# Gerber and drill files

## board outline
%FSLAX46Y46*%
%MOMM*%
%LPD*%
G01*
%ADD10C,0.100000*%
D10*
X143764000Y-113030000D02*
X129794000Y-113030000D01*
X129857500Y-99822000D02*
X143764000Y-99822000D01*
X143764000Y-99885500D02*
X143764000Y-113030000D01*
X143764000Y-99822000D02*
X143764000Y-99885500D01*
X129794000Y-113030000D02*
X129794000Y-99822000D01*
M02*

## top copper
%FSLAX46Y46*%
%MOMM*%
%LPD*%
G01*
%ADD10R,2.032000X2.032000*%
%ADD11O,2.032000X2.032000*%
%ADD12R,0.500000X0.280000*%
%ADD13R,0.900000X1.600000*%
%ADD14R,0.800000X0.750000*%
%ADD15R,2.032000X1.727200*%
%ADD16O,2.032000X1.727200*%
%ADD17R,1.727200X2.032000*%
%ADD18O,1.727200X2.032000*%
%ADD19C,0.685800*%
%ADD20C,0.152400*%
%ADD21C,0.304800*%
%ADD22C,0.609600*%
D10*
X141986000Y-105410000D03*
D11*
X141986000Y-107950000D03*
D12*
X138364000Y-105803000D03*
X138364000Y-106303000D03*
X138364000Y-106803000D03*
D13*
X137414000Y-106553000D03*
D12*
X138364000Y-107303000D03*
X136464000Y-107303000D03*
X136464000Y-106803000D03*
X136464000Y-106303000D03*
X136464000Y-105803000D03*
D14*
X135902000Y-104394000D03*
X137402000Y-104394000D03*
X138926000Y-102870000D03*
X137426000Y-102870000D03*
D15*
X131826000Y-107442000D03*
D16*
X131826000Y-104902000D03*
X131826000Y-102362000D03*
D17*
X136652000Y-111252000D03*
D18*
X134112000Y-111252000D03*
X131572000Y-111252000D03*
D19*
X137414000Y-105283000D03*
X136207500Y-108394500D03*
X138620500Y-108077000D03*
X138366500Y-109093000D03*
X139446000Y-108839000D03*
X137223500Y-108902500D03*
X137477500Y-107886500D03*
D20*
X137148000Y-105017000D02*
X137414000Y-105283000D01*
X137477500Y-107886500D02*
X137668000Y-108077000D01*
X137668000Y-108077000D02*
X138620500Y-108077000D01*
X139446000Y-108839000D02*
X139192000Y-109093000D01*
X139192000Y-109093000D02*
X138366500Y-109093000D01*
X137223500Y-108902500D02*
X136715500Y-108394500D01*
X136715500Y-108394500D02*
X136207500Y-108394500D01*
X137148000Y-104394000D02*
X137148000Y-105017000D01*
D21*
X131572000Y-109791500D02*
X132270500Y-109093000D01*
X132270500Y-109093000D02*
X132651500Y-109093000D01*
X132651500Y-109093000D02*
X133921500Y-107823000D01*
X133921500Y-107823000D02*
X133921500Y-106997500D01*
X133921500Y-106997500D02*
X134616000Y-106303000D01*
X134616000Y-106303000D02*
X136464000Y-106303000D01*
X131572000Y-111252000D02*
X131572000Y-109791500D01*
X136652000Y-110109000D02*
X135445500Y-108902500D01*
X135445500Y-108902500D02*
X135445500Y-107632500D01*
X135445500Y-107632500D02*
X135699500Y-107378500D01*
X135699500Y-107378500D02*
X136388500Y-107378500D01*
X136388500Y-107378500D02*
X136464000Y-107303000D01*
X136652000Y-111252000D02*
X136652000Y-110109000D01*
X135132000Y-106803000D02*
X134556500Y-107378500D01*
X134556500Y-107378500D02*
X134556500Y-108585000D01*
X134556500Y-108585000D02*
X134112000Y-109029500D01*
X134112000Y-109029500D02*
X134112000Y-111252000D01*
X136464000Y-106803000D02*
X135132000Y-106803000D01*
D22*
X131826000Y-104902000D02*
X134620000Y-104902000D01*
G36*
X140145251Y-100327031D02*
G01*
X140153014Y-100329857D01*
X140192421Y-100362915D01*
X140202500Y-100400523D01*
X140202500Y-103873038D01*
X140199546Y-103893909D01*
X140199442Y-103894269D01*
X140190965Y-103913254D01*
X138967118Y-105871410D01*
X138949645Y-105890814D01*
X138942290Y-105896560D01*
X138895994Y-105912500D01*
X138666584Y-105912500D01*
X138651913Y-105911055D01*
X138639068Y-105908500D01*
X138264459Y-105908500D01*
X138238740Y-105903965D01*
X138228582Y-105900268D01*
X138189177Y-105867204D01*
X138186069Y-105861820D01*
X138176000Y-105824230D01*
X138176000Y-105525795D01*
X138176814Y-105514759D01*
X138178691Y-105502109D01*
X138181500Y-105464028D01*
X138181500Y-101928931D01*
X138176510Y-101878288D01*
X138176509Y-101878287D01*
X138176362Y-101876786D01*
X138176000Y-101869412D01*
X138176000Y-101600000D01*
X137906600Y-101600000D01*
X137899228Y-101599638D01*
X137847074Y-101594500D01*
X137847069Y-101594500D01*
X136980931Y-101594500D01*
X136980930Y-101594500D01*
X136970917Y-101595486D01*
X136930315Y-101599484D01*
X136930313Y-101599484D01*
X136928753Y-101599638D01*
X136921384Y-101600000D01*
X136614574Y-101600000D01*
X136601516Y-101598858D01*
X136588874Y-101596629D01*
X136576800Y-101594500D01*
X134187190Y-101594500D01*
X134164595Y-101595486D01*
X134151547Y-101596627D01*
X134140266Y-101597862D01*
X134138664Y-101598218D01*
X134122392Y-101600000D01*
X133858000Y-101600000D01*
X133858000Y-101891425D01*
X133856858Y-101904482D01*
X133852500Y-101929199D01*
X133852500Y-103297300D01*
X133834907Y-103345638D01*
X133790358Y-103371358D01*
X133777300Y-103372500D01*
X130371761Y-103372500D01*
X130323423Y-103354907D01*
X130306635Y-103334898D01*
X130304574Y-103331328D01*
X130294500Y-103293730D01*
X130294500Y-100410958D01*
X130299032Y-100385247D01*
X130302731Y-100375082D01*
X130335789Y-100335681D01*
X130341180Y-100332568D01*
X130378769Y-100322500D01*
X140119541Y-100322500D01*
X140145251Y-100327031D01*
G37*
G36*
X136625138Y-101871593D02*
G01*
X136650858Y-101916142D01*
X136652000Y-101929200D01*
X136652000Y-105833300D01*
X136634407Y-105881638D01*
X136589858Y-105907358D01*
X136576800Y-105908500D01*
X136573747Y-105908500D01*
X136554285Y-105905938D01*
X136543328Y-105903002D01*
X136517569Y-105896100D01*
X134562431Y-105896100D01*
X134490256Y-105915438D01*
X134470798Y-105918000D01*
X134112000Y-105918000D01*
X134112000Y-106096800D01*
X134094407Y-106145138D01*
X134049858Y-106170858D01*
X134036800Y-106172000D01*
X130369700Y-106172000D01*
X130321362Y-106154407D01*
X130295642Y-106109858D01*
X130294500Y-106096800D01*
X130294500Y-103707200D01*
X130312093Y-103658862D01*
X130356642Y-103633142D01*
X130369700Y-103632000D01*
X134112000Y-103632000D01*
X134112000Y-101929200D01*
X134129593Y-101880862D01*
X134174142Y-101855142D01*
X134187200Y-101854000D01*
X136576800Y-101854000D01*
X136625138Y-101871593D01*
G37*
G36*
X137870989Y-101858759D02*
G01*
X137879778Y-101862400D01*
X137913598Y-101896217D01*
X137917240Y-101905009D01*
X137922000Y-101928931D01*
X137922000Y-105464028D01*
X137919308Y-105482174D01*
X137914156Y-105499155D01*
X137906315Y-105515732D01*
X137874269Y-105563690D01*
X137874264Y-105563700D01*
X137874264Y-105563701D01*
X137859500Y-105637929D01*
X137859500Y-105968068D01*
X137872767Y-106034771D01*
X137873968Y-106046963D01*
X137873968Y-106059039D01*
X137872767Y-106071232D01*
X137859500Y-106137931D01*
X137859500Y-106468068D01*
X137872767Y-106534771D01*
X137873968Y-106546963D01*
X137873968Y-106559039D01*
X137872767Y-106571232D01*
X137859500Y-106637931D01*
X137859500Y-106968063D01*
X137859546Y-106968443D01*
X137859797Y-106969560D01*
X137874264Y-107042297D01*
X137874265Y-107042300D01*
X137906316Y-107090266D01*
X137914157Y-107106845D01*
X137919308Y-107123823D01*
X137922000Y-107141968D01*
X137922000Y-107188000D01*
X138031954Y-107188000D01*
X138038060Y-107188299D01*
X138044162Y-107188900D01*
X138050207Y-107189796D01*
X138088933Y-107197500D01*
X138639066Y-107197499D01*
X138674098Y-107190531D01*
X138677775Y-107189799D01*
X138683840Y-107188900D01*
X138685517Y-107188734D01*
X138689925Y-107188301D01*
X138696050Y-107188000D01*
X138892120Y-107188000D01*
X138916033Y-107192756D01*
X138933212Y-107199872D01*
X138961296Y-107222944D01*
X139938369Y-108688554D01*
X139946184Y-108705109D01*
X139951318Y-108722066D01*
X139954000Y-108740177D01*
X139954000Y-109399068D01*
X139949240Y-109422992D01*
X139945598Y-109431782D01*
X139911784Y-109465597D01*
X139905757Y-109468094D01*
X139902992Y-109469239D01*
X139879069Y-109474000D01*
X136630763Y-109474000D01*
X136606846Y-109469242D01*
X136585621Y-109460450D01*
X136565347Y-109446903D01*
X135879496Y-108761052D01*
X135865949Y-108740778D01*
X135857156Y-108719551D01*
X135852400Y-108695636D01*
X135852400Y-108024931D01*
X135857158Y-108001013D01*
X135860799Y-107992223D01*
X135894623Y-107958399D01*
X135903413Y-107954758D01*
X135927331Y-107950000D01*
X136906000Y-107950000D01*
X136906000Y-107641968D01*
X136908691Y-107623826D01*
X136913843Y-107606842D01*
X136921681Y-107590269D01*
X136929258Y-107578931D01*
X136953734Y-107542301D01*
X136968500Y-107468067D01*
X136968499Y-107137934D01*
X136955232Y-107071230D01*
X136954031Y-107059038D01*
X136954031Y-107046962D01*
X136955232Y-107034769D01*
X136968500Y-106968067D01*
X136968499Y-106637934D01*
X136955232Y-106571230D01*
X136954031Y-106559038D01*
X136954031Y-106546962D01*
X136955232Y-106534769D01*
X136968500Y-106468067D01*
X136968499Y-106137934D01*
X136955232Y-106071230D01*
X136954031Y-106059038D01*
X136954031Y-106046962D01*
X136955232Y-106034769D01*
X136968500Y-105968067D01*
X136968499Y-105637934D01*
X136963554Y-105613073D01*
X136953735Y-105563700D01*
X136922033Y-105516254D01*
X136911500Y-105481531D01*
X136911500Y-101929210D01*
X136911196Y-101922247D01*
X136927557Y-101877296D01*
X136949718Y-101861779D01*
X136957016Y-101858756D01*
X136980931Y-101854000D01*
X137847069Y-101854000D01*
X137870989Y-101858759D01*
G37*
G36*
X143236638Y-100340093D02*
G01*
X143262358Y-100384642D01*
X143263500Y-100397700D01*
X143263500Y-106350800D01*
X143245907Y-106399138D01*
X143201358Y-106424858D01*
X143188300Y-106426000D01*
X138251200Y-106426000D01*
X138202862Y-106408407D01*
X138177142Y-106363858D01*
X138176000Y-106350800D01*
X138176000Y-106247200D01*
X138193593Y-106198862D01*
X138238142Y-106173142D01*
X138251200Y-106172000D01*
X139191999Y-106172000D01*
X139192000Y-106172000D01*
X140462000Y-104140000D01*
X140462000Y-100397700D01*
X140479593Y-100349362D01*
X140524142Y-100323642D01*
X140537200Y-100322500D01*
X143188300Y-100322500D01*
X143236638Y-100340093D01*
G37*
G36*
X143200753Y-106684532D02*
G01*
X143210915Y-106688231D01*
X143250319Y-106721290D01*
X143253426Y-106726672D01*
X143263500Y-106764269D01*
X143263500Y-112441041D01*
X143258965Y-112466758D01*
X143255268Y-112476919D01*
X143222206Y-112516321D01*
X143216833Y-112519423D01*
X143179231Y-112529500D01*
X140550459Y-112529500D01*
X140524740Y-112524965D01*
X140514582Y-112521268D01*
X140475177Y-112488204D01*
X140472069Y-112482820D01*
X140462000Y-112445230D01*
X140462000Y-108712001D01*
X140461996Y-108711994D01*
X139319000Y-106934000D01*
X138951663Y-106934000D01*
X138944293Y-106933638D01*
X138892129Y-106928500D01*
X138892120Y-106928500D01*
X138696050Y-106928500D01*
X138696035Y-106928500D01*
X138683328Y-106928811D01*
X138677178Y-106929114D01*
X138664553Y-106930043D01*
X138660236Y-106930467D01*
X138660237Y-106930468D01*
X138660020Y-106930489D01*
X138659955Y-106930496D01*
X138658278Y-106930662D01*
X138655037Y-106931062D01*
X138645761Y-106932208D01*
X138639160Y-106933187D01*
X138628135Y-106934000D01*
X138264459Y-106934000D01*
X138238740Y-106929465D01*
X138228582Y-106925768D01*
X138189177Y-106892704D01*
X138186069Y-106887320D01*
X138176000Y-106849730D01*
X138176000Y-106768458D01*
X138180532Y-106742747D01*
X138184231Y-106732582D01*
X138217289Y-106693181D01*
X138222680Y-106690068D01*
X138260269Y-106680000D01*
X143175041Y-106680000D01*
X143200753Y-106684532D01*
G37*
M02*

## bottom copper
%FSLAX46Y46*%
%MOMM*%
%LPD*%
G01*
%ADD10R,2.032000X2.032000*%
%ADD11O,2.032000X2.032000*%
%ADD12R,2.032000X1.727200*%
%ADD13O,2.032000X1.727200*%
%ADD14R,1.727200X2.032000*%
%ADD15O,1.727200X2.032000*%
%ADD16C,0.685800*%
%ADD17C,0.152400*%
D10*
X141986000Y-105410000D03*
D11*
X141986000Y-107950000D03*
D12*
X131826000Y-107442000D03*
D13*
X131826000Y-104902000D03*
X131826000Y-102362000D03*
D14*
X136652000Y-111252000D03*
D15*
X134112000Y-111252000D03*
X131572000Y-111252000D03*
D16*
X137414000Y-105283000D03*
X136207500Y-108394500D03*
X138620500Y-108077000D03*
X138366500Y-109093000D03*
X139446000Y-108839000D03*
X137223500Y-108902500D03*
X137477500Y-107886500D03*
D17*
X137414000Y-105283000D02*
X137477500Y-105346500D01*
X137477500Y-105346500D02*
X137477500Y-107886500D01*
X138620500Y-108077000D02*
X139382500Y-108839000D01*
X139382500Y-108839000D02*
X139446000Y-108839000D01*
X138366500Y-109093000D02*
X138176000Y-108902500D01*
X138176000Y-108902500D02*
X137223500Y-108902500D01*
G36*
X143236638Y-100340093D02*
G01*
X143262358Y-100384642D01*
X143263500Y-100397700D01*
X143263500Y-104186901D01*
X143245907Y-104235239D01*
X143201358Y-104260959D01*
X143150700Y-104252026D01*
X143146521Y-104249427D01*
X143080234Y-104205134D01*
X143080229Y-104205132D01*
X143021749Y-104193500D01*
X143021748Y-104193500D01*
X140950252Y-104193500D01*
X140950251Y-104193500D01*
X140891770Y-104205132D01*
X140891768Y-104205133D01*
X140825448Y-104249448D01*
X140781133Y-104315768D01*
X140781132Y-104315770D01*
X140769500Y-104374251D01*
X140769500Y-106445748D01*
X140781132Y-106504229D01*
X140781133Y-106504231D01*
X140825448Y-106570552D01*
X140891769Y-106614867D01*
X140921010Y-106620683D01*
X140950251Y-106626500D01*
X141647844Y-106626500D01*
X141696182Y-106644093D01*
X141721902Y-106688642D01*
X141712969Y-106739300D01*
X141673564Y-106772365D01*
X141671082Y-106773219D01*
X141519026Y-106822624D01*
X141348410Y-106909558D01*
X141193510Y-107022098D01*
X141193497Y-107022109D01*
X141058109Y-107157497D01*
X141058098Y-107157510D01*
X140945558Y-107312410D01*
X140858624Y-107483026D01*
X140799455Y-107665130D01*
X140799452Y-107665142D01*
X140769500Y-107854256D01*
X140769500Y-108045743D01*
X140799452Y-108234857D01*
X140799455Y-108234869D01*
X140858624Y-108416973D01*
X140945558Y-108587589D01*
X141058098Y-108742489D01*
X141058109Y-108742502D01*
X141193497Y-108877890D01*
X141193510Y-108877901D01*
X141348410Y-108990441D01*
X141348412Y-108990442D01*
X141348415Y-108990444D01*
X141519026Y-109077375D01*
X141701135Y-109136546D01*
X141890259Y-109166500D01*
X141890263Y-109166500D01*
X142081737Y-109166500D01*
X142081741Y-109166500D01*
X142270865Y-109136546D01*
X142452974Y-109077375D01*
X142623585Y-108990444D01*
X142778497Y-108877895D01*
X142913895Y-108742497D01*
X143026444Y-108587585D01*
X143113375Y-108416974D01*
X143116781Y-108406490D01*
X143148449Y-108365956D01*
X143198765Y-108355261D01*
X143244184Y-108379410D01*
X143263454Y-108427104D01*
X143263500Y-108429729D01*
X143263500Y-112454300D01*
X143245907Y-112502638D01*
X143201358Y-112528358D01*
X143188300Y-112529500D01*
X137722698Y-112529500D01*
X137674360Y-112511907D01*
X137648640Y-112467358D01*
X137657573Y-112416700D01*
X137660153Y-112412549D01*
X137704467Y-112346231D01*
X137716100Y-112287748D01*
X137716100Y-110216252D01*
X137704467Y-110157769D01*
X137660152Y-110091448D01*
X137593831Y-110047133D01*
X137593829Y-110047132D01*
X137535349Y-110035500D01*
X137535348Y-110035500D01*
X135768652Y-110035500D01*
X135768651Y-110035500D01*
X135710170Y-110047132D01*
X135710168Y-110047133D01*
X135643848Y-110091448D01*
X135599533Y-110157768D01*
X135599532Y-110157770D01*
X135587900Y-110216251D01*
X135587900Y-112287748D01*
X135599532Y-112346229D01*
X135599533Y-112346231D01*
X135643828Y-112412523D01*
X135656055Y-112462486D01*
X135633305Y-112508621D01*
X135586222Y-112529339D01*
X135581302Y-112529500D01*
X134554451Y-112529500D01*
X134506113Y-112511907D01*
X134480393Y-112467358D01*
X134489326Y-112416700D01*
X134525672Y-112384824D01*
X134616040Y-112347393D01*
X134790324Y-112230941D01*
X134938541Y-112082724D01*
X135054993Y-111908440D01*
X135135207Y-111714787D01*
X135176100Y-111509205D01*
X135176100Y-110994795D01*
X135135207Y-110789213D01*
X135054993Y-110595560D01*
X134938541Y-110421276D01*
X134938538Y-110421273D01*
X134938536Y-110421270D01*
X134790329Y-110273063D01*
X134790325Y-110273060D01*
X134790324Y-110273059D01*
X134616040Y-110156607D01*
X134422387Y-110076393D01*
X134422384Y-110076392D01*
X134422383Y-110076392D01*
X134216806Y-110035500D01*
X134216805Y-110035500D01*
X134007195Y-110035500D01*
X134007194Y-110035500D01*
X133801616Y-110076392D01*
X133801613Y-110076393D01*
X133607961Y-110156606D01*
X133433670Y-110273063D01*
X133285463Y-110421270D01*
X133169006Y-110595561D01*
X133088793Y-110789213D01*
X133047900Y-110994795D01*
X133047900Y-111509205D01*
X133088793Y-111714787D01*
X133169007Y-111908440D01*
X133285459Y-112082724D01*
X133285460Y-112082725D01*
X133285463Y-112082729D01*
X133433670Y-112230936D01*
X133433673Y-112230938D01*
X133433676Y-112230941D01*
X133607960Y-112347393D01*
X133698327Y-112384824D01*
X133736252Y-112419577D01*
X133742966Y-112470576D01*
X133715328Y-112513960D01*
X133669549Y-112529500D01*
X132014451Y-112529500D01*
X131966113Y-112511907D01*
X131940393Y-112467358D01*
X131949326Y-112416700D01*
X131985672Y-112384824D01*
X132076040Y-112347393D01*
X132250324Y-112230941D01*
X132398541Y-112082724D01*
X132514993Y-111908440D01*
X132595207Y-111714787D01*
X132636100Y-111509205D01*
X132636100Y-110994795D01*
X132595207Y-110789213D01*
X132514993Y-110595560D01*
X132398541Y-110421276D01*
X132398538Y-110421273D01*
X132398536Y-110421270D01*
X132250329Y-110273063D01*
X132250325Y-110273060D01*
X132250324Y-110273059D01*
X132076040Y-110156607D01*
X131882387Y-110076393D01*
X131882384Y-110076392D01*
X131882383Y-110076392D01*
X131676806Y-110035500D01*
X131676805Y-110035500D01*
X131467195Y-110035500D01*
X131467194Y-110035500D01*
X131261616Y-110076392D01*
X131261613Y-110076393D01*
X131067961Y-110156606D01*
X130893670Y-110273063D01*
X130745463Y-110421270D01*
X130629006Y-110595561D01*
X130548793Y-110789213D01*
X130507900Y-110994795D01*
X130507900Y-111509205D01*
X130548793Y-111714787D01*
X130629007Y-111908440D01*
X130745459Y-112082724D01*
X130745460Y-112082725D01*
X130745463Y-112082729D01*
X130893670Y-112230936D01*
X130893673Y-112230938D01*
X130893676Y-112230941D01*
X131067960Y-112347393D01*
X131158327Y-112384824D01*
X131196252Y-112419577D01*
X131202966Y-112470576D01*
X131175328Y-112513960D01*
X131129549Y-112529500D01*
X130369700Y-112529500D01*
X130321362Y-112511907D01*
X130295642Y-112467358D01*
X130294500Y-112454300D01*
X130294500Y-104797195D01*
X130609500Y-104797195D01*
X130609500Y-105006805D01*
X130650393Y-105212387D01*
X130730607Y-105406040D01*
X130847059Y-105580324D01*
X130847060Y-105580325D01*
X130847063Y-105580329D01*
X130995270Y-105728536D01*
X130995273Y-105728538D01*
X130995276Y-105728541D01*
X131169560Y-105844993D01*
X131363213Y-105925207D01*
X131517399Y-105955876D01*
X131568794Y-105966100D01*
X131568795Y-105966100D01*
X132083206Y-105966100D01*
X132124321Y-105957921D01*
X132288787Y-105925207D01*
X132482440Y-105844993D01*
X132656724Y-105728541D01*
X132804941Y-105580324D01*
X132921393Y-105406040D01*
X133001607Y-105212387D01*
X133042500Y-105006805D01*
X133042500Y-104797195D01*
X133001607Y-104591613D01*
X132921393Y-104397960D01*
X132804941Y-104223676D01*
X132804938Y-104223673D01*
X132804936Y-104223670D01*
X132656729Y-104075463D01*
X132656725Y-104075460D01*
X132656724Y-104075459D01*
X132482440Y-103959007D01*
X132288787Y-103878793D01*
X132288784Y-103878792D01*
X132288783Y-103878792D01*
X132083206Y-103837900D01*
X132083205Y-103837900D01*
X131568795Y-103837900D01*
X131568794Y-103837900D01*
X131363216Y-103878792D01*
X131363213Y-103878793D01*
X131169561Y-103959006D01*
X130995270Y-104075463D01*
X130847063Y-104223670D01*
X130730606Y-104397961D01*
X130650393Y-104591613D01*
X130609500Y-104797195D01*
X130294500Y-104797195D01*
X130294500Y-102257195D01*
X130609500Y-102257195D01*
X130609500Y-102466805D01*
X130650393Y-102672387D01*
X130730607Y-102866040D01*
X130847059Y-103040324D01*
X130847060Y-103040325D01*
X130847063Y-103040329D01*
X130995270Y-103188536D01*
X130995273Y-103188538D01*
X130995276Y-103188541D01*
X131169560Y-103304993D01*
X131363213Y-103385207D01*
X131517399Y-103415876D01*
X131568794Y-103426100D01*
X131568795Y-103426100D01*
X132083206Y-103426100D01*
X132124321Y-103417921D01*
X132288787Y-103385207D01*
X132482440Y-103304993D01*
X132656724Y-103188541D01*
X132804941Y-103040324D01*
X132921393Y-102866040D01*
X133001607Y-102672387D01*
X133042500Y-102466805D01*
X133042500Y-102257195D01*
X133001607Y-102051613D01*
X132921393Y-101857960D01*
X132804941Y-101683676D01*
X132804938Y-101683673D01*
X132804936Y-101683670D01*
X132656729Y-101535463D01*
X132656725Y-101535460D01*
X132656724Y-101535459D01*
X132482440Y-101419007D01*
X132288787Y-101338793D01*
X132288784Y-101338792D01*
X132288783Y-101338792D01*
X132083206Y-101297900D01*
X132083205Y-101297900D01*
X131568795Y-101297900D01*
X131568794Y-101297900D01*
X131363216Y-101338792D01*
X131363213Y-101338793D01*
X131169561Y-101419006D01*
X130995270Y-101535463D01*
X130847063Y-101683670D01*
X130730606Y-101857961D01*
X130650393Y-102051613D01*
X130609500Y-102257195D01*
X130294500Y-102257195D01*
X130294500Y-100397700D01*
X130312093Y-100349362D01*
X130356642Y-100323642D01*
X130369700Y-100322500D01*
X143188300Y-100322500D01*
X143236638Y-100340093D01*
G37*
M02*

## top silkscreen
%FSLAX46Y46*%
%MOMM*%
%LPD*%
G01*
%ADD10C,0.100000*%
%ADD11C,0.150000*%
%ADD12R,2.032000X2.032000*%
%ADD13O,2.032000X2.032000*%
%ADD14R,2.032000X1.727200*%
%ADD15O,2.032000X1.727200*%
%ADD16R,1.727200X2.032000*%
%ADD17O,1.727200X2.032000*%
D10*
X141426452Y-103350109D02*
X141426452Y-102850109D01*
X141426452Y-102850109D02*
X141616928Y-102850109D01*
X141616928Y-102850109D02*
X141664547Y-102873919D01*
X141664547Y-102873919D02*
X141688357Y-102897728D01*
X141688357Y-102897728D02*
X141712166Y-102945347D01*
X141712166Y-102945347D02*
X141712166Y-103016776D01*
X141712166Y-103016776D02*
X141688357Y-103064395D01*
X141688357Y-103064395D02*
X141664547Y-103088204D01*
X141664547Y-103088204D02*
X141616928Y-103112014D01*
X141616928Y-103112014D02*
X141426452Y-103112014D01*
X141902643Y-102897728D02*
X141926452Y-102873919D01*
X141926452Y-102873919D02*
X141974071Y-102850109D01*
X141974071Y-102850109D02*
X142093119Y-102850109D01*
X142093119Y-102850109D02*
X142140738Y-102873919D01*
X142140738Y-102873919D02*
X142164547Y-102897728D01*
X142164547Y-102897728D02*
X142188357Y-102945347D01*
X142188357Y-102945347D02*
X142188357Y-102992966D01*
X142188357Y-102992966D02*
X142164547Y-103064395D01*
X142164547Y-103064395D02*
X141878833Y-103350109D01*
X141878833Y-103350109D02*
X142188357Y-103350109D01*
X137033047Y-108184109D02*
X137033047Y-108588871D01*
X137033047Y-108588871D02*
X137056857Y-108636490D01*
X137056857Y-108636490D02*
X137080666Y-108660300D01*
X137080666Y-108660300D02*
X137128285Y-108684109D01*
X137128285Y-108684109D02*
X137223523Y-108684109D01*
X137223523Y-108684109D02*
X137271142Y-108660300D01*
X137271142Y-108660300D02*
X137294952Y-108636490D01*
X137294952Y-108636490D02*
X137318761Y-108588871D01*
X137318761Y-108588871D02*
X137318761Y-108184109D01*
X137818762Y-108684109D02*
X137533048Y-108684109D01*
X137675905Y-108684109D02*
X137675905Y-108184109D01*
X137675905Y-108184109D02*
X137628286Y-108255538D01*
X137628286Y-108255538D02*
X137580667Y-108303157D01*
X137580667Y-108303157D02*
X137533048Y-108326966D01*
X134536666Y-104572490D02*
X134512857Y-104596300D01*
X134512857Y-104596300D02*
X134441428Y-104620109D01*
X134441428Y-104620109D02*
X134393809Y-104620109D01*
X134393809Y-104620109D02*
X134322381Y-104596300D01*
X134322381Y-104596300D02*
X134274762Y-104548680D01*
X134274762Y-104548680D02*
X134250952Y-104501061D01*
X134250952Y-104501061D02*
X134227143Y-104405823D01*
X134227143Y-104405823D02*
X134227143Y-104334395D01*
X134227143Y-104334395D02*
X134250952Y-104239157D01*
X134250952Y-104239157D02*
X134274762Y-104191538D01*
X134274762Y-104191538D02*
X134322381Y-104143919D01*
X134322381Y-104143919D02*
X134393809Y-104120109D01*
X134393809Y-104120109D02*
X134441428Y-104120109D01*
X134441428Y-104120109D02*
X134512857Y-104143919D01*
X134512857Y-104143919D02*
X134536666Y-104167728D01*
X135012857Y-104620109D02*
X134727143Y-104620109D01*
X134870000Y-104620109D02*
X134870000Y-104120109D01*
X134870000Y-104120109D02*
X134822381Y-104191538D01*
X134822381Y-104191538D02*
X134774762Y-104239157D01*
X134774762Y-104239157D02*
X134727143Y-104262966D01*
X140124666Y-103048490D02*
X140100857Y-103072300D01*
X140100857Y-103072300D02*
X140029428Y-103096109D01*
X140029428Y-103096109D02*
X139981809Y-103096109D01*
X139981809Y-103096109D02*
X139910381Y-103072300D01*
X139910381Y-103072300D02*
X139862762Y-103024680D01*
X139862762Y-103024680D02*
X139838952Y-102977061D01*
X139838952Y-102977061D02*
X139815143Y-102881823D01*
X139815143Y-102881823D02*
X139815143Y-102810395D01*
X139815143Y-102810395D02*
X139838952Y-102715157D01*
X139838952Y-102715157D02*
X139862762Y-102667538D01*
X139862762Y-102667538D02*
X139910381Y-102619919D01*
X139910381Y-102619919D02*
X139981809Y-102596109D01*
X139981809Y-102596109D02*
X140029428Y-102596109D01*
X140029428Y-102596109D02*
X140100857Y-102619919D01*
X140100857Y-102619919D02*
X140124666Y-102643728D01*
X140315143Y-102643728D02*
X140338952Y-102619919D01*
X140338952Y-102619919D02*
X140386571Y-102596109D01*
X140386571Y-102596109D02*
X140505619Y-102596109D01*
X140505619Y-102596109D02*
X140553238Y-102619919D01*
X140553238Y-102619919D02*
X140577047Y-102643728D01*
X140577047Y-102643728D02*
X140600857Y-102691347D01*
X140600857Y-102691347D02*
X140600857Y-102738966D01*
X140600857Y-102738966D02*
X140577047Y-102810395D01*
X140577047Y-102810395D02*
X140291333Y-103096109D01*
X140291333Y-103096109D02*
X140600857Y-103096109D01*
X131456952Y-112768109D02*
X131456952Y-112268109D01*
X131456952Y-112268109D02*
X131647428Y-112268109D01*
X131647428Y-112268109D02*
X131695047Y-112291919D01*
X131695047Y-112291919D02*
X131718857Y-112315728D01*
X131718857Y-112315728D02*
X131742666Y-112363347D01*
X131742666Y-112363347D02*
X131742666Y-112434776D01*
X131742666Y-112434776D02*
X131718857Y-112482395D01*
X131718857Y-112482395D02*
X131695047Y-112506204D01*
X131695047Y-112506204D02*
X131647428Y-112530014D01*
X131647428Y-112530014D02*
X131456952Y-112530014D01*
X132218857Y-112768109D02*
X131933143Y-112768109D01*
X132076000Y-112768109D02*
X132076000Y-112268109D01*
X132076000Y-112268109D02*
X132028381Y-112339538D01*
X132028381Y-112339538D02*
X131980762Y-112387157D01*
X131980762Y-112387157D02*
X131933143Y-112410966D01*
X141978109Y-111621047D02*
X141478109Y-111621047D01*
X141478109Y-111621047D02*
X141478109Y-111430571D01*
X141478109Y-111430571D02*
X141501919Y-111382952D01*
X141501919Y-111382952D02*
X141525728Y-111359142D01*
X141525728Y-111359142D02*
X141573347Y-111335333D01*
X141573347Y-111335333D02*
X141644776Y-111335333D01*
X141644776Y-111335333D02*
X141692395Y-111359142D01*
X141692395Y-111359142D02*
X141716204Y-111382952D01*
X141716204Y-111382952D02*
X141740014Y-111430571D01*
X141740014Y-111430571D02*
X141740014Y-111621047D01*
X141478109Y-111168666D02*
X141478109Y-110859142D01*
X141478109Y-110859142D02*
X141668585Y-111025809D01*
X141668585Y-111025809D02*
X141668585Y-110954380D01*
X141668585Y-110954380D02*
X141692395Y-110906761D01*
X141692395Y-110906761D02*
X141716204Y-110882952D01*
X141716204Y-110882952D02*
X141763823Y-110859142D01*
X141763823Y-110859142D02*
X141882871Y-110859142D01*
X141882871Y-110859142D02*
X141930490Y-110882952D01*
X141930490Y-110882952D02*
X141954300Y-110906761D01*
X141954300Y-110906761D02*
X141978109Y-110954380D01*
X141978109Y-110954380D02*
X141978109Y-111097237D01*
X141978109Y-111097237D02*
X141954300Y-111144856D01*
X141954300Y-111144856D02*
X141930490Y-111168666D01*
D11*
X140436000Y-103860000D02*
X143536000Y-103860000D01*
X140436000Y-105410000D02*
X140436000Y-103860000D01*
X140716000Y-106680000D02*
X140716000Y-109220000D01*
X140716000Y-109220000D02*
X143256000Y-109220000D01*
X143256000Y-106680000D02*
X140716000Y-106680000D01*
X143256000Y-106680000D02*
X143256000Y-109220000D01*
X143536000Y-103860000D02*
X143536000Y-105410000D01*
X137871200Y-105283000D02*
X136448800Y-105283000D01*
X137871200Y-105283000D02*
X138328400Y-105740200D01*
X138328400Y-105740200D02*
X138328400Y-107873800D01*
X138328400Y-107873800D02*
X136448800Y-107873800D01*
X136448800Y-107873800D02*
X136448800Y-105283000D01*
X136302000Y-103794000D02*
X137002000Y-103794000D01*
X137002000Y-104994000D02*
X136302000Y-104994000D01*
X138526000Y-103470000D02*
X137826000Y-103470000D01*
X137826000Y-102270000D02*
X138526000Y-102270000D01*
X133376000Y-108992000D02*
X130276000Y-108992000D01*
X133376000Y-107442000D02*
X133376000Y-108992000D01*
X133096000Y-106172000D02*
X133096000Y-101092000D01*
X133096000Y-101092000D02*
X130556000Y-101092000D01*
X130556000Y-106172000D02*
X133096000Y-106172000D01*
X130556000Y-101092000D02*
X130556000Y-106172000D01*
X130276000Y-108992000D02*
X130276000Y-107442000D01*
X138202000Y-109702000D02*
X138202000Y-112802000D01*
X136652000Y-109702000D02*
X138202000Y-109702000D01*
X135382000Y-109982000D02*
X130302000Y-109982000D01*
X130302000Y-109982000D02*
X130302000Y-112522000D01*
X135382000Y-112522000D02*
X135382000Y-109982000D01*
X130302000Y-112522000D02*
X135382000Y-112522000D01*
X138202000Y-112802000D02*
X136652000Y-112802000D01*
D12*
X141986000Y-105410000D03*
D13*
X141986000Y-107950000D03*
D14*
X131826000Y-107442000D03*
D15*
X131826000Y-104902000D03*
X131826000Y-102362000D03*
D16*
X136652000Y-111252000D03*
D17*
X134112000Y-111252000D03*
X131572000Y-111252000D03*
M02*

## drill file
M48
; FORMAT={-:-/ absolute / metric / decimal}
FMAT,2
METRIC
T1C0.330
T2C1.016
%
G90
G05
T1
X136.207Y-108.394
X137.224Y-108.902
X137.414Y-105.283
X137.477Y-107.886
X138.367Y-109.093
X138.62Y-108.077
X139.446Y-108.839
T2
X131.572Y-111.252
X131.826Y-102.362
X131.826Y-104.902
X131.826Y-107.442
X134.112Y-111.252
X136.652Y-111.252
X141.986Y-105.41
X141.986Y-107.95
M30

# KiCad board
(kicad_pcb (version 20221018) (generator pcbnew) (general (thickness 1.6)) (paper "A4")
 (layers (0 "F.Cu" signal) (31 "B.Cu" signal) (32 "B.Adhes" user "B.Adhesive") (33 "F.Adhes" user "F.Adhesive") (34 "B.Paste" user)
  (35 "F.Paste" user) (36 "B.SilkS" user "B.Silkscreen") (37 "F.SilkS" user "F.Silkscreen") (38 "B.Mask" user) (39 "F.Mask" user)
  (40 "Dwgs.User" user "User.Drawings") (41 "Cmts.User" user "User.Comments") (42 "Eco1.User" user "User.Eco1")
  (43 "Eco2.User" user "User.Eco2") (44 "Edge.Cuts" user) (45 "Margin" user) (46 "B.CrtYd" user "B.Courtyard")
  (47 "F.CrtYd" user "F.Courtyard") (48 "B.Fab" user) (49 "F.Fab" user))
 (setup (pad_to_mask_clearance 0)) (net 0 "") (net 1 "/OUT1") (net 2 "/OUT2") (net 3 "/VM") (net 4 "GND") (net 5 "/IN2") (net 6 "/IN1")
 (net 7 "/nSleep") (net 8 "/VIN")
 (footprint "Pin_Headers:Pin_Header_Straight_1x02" (layer "F.Cu") (at 141.986 105.41)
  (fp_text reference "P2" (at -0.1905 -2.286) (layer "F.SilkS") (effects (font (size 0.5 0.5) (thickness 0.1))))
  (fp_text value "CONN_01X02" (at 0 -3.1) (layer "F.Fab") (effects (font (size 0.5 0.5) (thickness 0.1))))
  (fp_line (start -1.55 -1.55) (end 1.55 -1.55) (stroke (width 0.15) (type solid)) (layer "F.SilkS"))
  (fp_line (start -1.55 0) (end -1.55 -1.55) (stroke (width 0.15) (type solid)) (layer "F.SilkS"))
  (fp_line (start -1.27 1.27) (end -1.27 3.81) (stroke (width 0.15) (type solid)) (layer "F.SilkS"))
  (fp_line (start -1.27 3.81) (end 1.27 3.81) (stroke (width 0.15) (type solid)) (layer "F.SilkS"))
  (fp_line (start 1.27 1.27) (end -1.27 1.27) (stroke (width 0.15) (type solid)) (layer "F.SilkS"))
  (fp_line (start 1.27 1.27) (end 1.27 3.81) (stroke (width 0.15) (type solid)) (layer "F.SilkS"))
  (fp_line (start 1.55 -1.55) (end 1.55 0) (stroke (width 0.15) (type solid)) (layer "F.SilkS"))
  (pad "1" thru_hole rect (at 0 0) (size 2.032 2.032) (drill 1.016) (layers "*.Cu" "*.Mask" "F.SilkS") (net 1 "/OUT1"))
  (pad "2" thru_hole oval (at 0 2.54) (size 2.032 2.032) (drill 1.016) (layers "*.Cu" "*.Mask" "F.SilkS") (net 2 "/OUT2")))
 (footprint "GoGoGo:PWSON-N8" (layer "F.Cu") (at 137.414 106.553 -90)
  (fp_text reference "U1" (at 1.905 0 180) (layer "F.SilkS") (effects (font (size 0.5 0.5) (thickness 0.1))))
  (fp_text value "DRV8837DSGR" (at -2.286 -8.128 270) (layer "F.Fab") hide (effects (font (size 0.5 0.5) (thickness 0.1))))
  (fp_line (start -1.27 -0.4572) (end -1.27 0.9652) (stroke (width 0.15) (type solid)) (layer "F.SilkS"))
  (fp_line (start -1.27 -0.4572) (end -0.8128 -0.9144) (stroke (width 0.15) (type solid)) (layer "F.SilkS"))
  (fp_line (start -0.8128 -0.9144) (end 1.3208 -0.9144) (stroke (width 0.15) (type solid)) (layer "F.SilkS"))
  (fp_line (start 1.3208 -0.9144) (end 1.3208 0.9652) (stroke (width 0.15) (type solid)) (layer "F.SilkS"))
  (fp_line (start 1.3208 0.9652) (end -1.27 0.9652) (stroke (width 0.15) (type solid)) (layer "F.SilkS"))
  (pad "1" smd rect (at -0.75 -0.95 270) (size 0.28 0.5) (layers "F.Cu" "F.Paste" "F.Mask") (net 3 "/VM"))
  (pad "2" smd rect (at -0.25 -0.95 270) (size 0.28 0.5) (layers "F.Cu" "F.Paste" "F.Mask") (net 1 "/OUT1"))
  (pad "3" smd rect (at 0.25 -0.95 270) (size 0.28 0.5) (layers "F.Cu" "F.Paste" "F.Mask") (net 2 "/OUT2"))
  (pad "4" smd rect (at 0 0 270) (size 1.6 0.9) (layers "F.Cu" "F.Paste" "F.Mask") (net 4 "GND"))
  (pad "4" smd rect (at 0.75 -0.95 270) (size 0.28 0.5) (layers "F.Cu" "F.Paste" "F.Mask") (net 4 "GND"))
  (pad "5" smd rect (at 0.75 0.95 270) (size 0.28 0.5) (layers "F.Cu" "F.Paste" "F.Mask") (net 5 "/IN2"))
  (pad "6" smd rect (at 0.25 0.95 270) (size 0.28 0.5) (layers "F.Cu" "F.Paste" "F.Mask") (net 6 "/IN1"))
  (pad "7" smd rect (at -0.25 0.95 270) (size 0.28 0.5) (layers "F.Cu" "F.Paste" "F.Mask") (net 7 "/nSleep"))
  (pad "8" smd rect (at -0.75 0.95 270) (size 0.28 0.5) (layers "F.Cu" "F.Paste" "F.Mask") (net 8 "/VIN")))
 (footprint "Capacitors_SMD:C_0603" (layer "F.Cu") (at 136.652 104.394)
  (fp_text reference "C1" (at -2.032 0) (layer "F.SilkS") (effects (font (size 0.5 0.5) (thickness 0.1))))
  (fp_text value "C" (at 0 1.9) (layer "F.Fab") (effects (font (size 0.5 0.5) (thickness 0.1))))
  (fp_line (start -0.35 -0.6) (end 0.35 -0.6) (stroke (width 0.15) (type solid)) (layer "F.SilkS"))
  (fp_line (start 0.35 0.6) (end -0.35 0.6) (stroke (width 0.15) (type solid)) (layer "F.SilkS"))
  (pad "1" smd rect (at -0.75 0) (size 0.8 0.75) (layers "F.Cu" "F.Paste" "F.Mask") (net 8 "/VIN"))
  (pad "2" smd rect (at 0.75 0) (size 0.8 0.75) (layers "F.Cu" "F.Paste" "F.Mask") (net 4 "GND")))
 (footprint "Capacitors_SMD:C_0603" (layer "F.Cu") (at 138.176 102.87 180)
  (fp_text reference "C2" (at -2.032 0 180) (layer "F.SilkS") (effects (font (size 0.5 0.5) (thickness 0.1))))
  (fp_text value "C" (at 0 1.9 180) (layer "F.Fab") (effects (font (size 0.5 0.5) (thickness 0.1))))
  (fp_line (start -0.35 -0.6) (end 0.35 -0.6) (stroke (width 0.15) (type solid)) (layer "F.SilkS"))
  (fp_line (start 0.35 0.6) (end -0.35 0.6) (stroke (width 0.15) (type solid)) (layer "F.SilkS"))
  (pad "1" smd rect (at -0.75 0 180) (size 0.8 0.75) (layers "F.Cu" "F.Paste" "F.Mask") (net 3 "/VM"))
  (pad "2" smd rect (at 0.75 0 180) (size 0.8 0.75) (layers "F.Cu" "F.Paste" "F.Mask") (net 4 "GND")))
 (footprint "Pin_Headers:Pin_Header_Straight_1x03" (layer "F.Cu") (at 131.826 107.442 180)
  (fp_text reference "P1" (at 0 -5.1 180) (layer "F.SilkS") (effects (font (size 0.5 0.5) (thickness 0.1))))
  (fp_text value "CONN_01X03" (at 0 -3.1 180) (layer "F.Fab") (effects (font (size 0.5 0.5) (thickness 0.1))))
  (fp_line (start -1.55 -1.55) (end 1.55 -1.55) (stroke (width 0.15) (type solid)) (layer "F.SilkS"))
  (fp_line (start -1.55 0) (end -1.55 -1.55) (stroke (width 0.15) (type solid)) (layer "F.SilkS"))
  (fp_line (start -1.27 1.27) (end -1.27 6.35) (stroke (width 0.15) (type solid)) (layer "F.SilkS"))
  (fp_line (start -1.27 6.35) (end 1.27 6.35) (stroke (width 0.15) (type solid)) (layer "F.SilkS"))
  (fp_line (start 1.27 1.27) (end -1.27 1.27) (stroke (width 0.15) (type solid)) (layer "F.SilkS"))
  (fp_line (start 1.27 6.35) (end 1.27 1.27) (stroke (width 0.15) (type solid)) (layer "F.SilkS"))
  (fp_line (start 1.55 -1.55) (end 1.55 0) (stroke (width 0.15) (type solid)) (layer "F.SilkS"))
  (pad "1" thru_hole rect (at 0 0 180) (size 2.032 1.7272) (drill 1.016) (layers "*.Cu" "*.Mask" "F.SilkS") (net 4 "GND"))
  (pad "2" thru_hole oval (at 0 2.54 180) (size 2.032 1.7272) (drill 1.016) (layers "*.Cu" "*.Mask" "F.SilkS") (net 8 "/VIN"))
  (pad "3" thru_hole oval (at 0 5.08 180) (size 2.032 1.7272) (drill 1.016) (layers "*.Cu" "*.Mask" "F.SilkS") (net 3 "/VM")))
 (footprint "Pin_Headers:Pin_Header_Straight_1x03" (layer "F.Cu") (at 136.652 111.252 -90)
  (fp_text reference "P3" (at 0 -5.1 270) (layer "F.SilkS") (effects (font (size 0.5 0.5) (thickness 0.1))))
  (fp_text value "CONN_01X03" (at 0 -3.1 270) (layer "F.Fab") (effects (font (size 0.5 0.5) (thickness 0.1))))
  (fp_line (start -1.55 -1.55) (end 1.55 -1.55) (stroke (width 0.15) (type solid)) (layer "F.SilkS"))
  (fp_line (start -1.55 0) (end -1.55 -1.55) (stroke (width 0.15) (type solid)) (layer "F.SilkS"))
  (fp_line (start -1.27 1.27) (end -1.27 6.35) (stroke (width 0.15) (type solid)) (layer "F.SilkS"))
  (fp_line (start -1.27 6.35) (end 1.27 6.35) (stroke (width 0.15) (type solid)) (layer "F.SilkS"))
  (fp_line (start 1.27 1.27) (end -1.27 1.27) (stroke (width 0.15) (type solid)) (layer "F.SilkS"))
  (fp_line (start 1.27 6.35) (end 1.27 1.27) (stroke (width 0.15) (type solid)) (layer "F.SilkS"))
  (fp_line (start 1.55 -1.55) (end 1.55 0) (stroke (width 0.15) (type solid)) (layer "F.SilkS"))
  (pad "1" thru_hole rect (at 0 0 270) (size 2.032 1.7272) (drill 1.016) (layers "*.Cu" "*.Mask" "F.SilkS") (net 5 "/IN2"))
  (pad "2" thru_hole oval (at 0 2.54 270) (size 2.032 1.7272) (drill 1.016) (layers "*.Cu" "*.Mask" "F.SilkS") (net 6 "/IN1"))
  (pad "3" thru_hole oval (at 0 5.08 270) (size 2.032 1.7272) (drill 1.016) (layers "*.Cu" "*.Mask" "F.SilkS") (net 7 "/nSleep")))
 (gr_line (start 143.764 113.03) (end 129.794 113.03) (stroke (width 0.1) (type solid)) (layer "Edge.Cuts"))
 (gr_line (start 129.8575 99.822) (end 143.764 99.822) (stroke (width 0.1) (type solid)) (layer "Edge.Cuts"))
 (gr_line (start 143.764 99.8855) (end 143.764 113.03) (stroke (width 0.1) (type solid)) (layer "Edge.Cuts"))
 (gr_line (start 143.764 99.822) (end 143.764 99.8855) (stroke (width 0.1) (type solid)) (layer "Edge.Cuts"))
 (gr_line (start 129.794 113.03) (end 129.794 99.822) (stroke (width 0.1) (type solid)) (layer "Edge.Cuts"))
 (segment (start 137.148 105.017) (end 137.414 105.283) (width 0.1524) (layer "F.Cu") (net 4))
 (segment (start 137.4775 107.8865) (end 137.668 108.077) (width 0.1524) (layer "F.Cu") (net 4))
 (segment (start 137.668 108.077) (end 138.6205 108.077) (width 0.1524) (layer "F.Cu") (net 4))
 (segment (start 139.446 108.839) (end 139.192 109.093) (width 0.1524) (layer "F.Cu") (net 4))
 (segment (start 139.192 109.093) (end 138.3665 109.093) (width 0.1524) (layer "F.Cu") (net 4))
 (segment (start 137.2235 108.9025) (end 136.7155 108.3945) (width 0.1524) (layer "F.Cu") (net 4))
 (segment (start 136.7155 108.3945) (end 136.2075 108.3945) (width 0.1524) (layer "F.Cu") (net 4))
 (segment (start 137.148 104.394) (end 137.148 105.017) (width 0.1524) (layer "F.Cu") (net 4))
 (via (at 137.414 105.283) (size 0.6858) (drill 0.3302) (layers "F.Cu" "B.Cu") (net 4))
 (via (at 136.2075 108.3945) (size 0.6858) (drill 0.3302) (layers "F.Cu" "B.Cu") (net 4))
 (via (at 138.6205 108.077) (size 0.6858) (drill 0.3302) (layers "F.Cu" "B.Cu") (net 4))
 (via (at 138.3665 109.093) (size 0.6858) (drill 0.3302) (layers "F.Cu" "B.Cu") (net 4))
 (via (at 139.446 108.839) (size 0.6858) (drill 0.3302) (layers "F.Cu" "B.Cu") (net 4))
 (via (at 137.2235 108.9025) (size 0.6858) (drill 0.3302) (layers "F.Cu" "B.Cu") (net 4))
 (via (at 137.4775 107.8865) (size 0.6858) (drill 0.3302) (layers "F.Cu" "B.Cu") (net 4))
 (segment (start 137.414 105.283) (end 137.4775 105.3465) (width 0.1524) (layer "B.Cu") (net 4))
 (segment (start 137.4775 105.3465) (end 137.4775 107.8865) (width 0.1524) (layer "B.Cu") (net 4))
 (segment (start 138.6205 108.077) (end 139.3825 108.839) (width 0.1524) (layer "B.Cu") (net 4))
 (segment (start 139.3825 108.839) (end 139.446 108.839) (width 0.1524) (layer "B.Cu") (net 4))
 (segment (start 138.3665 109.093) (end 138.176 108.9025) (width 0.1524) (layer "B.Cu") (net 4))
 (segment (start 138.176 108.9025) (end 137.2235 108.9025) (width 0.1524) (layer "B.Cu") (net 4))
 (segment (start 131.572 109.7915) (end 132.2705 109.093) (width 0.3048) (layer "F.Cu") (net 7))
 (segment (start 132.2705 109.093) (end 132.6515 109.093) (width 0.3048) (layer "F.Cu") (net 7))
 (segment (start 132.6515 109.093) (end 133.9215 107.823) (width 0.3048) (layer "F.Cu") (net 7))
 (segment (start 133.9215 107.823) (end 133.9215 106.9975) (width 0.3048) (layer "F.Cu") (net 7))
 (segment (start 133.9215 106.9975) (end 134.616 106.303) (width 0.3048) (layer "F.Cu") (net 7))
 (segment (start 134.616 106.303) (end 136.464 106.303) (width 0.3048) (layer "F.Cu") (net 7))
 (segment (start 131.572 111.252) (end 131.572 109.7915) (width 0.3048) (layer "F.Cu") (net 7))
 (segment (start 136.652 110.109) (end 135.4455 108.9025) (width 0.3048) (layer "F.Cu") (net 5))
 (segment (start 135.4455 108.9025) (end 135.4455 107.6325) (width 0.3048) (layer "F.Cu") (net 5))
 (segment (start 135.4455 107.6325) (end 135.6995 107.3785) (width 0.3048) (layer "F.Cu") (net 5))
 (segment (start 135.6995 107.3785) (end 136.3885 107.3785) (width 0.3048) (layer "F.Cu") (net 5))
 (segment (start 136.3885 107.3785) (end 136.464 107.303) (width 0.3048) (layer "F.Cu") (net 5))
 (segment (start 136.652 111.252) (end 136.652 110.109) (width 0.3048) (layer "F.Cu") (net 5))
 (segment (start 135.132 106.803) (end 134.5565 107.3785) (width 0.3048) (layer "F.Cu") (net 6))
 (segment (start 134.5565 107.3785) (end 134.5565 108.585) (width 0.3048) (layer "F.Cu") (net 6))
 (segment (start 134.5565 108.585) (end 134.112 109.0295) (width 0.3048) (layer "F.Cu") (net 6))
 (segment (start 134.112 109.0295) (end 134.112 111.252) (width 0.3048) (layer "F.Cu") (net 6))
 (segment (start 136.464 106.803) (end 135.132 106.803) (width 0.3048) (layer "F.Cu") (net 6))
 (segment (start 131.826 104.902) (end 134.62 104.902) (width 0.6096) (layer "F.Cu") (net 8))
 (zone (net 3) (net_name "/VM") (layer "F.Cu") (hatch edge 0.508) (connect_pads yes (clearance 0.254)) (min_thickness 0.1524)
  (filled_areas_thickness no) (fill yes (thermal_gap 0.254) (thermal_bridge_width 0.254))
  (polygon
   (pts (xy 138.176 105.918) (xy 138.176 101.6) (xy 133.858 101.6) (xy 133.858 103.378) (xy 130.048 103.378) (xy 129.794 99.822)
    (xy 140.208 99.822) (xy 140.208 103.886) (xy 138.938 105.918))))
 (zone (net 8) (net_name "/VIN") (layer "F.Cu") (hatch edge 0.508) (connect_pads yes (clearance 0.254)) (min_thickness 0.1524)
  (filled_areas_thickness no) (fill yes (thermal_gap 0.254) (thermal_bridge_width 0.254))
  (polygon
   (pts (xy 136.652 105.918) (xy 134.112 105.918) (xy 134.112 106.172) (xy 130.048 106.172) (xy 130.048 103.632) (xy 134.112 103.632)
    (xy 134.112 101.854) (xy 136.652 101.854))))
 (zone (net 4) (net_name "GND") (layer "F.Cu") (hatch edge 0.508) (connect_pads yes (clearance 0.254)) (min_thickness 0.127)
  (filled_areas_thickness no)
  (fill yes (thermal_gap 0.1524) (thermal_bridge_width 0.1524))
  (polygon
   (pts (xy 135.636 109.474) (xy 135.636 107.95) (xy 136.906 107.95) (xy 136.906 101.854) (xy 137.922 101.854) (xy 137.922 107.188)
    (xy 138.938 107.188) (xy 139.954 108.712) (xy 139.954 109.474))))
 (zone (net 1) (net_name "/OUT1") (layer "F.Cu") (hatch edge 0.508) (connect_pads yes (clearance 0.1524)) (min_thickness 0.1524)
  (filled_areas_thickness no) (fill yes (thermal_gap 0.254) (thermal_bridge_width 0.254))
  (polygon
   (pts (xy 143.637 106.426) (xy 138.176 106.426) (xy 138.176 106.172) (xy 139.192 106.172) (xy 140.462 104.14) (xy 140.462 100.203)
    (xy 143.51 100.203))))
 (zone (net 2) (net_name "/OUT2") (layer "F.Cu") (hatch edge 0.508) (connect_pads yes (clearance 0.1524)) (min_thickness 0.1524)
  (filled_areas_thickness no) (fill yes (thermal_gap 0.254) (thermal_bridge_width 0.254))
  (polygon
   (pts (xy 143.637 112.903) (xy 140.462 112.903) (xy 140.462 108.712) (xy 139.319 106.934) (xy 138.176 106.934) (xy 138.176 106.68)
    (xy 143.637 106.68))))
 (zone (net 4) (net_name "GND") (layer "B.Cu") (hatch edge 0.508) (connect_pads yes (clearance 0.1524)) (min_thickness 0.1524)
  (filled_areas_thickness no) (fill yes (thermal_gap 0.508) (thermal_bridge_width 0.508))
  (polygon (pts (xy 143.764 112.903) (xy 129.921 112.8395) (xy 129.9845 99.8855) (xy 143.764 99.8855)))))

